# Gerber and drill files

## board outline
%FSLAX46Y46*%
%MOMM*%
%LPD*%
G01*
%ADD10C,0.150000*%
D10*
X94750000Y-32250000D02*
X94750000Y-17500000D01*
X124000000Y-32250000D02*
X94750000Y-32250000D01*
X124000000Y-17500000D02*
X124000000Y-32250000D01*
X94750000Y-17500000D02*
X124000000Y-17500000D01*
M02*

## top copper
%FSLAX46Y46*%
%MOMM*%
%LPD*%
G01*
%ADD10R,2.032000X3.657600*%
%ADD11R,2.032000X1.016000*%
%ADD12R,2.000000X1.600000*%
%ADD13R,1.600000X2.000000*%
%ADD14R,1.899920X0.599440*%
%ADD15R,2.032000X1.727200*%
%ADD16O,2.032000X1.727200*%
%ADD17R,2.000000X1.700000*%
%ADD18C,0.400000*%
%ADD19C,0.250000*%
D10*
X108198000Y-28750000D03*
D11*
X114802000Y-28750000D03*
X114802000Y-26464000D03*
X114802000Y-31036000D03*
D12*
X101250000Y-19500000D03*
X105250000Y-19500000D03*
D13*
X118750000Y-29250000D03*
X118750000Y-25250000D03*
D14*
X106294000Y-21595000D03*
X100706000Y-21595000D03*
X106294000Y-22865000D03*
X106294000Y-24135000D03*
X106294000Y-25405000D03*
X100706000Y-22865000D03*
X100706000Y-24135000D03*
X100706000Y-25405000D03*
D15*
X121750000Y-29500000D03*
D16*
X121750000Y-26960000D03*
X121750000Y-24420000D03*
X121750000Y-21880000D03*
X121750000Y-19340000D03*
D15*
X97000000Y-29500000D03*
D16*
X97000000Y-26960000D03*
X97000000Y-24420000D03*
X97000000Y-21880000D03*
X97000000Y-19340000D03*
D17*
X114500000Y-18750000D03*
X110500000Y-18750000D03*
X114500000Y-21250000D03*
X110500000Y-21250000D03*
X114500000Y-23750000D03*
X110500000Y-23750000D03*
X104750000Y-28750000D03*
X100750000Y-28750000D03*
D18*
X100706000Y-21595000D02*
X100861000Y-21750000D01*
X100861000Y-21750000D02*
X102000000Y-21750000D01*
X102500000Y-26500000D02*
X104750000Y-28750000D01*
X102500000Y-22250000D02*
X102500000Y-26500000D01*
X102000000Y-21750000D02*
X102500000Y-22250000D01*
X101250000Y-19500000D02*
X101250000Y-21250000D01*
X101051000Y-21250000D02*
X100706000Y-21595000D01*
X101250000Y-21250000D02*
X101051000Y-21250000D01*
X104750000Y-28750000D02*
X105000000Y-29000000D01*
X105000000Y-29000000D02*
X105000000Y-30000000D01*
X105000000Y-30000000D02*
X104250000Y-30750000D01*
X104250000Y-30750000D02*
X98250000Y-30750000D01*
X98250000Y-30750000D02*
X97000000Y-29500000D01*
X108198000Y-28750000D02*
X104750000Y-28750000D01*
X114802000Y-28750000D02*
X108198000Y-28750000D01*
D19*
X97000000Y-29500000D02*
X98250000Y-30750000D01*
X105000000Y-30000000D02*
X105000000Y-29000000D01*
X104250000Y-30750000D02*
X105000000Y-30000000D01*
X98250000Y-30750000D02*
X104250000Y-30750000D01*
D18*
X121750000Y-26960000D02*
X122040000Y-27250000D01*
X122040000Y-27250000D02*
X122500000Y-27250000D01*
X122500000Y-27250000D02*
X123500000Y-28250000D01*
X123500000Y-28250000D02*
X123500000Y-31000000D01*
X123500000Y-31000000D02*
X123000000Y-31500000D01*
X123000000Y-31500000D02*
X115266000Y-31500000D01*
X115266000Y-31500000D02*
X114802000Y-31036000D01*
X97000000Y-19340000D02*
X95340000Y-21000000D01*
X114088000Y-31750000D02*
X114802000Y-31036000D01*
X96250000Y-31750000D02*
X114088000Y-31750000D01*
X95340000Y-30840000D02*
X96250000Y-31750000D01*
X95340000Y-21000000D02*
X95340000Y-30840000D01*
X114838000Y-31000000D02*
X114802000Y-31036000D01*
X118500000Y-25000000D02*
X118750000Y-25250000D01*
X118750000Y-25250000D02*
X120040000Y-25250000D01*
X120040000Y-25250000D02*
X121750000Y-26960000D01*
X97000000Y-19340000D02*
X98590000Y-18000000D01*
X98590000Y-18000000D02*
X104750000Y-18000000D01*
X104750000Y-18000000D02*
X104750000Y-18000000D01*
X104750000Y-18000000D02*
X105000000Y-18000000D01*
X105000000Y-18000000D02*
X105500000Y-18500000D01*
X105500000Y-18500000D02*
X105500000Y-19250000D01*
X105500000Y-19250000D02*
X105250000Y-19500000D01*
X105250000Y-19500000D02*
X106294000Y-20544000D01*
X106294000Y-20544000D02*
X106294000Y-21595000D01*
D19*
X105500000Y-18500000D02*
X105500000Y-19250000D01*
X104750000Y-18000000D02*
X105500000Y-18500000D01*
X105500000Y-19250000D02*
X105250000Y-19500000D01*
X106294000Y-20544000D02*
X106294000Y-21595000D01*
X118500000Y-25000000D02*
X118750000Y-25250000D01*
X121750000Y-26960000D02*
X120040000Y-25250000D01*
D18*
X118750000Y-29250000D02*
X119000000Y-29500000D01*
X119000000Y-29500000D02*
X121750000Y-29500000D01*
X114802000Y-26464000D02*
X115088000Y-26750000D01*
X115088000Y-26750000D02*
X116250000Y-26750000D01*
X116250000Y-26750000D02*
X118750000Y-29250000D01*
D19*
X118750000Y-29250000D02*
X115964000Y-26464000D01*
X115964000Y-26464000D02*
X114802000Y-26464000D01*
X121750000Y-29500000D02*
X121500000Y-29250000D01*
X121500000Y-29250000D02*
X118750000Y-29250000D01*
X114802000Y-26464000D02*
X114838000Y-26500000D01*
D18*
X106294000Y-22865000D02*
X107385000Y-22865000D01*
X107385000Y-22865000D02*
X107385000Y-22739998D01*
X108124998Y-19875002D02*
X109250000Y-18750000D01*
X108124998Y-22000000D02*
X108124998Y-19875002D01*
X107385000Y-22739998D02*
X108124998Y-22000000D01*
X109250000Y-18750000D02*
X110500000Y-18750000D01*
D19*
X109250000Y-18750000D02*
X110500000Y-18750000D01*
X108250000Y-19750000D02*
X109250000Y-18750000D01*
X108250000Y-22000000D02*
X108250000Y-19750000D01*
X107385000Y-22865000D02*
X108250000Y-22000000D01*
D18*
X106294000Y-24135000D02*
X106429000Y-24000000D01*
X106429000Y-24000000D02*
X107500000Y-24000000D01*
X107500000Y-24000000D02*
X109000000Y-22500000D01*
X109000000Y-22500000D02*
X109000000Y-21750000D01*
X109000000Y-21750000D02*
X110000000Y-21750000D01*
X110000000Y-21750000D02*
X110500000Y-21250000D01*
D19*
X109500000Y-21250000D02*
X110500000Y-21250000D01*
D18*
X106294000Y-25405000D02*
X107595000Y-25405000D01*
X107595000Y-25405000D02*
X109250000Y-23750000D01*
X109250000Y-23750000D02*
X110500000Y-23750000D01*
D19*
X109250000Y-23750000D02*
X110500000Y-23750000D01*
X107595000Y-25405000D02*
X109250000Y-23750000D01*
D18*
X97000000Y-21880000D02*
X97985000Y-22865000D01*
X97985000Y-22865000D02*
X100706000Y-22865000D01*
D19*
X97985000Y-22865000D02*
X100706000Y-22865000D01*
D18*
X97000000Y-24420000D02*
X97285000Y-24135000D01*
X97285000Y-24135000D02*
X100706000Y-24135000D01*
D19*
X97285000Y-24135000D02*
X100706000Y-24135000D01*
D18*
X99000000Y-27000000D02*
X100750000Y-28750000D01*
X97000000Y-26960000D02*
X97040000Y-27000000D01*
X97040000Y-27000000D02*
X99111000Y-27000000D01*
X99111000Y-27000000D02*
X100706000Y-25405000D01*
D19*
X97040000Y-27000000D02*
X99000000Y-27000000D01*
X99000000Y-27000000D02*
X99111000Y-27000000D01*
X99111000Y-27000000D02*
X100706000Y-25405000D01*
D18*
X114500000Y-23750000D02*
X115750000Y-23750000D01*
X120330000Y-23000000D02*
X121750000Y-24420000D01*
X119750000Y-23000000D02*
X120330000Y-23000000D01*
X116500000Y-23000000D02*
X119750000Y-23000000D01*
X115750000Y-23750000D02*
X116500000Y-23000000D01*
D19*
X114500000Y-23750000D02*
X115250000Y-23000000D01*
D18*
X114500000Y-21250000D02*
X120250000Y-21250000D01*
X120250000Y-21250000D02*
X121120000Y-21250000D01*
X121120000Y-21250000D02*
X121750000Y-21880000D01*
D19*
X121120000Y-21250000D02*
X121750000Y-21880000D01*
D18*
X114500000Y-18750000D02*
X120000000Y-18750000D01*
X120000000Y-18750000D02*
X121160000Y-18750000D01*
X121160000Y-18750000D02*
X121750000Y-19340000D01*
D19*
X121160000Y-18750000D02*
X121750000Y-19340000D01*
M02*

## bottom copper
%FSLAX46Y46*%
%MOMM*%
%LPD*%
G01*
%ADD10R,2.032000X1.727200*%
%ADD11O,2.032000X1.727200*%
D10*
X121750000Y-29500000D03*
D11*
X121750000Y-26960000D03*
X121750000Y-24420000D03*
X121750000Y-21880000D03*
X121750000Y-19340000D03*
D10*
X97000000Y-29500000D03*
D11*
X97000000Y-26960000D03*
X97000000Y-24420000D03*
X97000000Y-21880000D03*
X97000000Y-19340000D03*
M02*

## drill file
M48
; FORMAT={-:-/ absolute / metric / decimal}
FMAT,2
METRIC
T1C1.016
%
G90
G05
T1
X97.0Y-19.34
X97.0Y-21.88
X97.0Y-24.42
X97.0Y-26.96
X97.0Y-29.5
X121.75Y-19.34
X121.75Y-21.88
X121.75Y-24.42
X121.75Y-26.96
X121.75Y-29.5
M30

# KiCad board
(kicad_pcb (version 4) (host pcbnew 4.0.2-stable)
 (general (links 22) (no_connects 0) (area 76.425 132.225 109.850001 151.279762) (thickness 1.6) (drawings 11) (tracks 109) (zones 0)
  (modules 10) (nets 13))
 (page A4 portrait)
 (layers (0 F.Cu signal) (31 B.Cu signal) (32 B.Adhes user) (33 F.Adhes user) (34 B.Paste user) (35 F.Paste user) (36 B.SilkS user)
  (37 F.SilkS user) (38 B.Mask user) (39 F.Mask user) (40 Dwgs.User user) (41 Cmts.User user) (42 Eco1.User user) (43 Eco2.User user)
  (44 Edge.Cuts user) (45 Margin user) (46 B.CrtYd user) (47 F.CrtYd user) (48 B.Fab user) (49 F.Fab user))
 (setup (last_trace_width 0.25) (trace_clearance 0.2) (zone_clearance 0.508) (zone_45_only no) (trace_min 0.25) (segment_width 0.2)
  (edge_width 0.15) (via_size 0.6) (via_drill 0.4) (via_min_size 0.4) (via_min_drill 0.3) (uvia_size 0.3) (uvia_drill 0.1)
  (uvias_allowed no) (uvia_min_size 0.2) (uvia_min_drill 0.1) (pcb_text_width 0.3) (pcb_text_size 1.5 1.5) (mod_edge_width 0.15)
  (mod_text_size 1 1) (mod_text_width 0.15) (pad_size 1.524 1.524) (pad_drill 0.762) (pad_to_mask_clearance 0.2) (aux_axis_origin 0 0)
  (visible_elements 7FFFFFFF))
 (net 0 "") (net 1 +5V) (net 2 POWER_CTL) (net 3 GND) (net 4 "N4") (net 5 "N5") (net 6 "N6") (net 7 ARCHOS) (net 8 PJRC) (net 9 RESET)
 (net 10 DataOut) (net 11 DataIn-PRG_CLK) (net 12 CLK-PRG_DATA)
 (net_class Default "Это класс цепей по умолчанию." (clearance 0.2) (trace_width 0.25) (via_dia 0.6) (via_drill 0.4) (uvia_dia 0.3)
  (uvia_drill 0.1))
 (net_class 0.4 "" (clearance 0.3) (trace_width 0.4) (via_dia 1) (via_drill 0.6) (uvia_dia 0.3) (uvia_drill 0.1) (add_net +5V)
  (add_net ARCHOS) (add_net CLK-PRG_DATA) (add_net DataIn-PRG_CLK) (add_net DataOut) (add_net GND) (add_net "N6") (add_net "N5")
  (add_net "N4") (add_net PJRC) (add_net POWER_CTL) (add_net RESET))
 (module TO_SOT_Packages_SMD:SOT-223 (layer F.Cu) (at 111.5 28.75 90)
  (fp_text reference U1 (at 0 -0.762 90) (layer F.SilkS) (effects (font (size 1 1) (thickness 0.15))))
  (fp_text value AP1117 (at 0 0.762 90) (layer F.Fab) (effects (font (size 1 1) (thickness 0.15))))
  (pad 2 smd rect (at 0 -3.302 90) (size 3.6576 2.032) (layers F.Cu F.Paste F.Mask) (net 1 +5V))
  (pad 2 smd rect (at 0 3.302 90) (size 1.016 2.032) (layers F.Cu F.Paste F.Mask) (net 1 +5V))
  (pad 3 smd rect (at 2.286 3.302 90) (size 1.016 2.032) (layers F.Cu F.Paste F.Mask) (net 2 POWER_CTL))
  (pad 1 smd rect (at -2.286 3.302 90) (size 1.016 2.032) (layers F.Cu F.Paste F.Mask) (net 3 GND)))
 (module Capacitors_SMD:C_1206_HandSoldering (layer F.Cu) (at 103.25 19.5)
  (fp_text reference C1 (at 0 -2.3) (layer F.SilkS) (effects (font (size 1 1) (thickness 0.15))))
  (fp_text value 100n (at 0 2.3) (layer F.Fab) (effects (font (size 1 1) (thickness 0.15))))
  (pad 1 smd rect (at -2 0) (size 2 1.6) (layers F.Cu F.Paste F.Mask) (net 1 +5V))
  (pad 2 smd rect (at 2 0) (size 2 1.6) (layers F.Cu F.Paste F.Mask) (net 3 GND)))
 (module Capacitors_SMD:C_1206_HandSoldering (layer F.Cu) (at 118.75 27.25 90)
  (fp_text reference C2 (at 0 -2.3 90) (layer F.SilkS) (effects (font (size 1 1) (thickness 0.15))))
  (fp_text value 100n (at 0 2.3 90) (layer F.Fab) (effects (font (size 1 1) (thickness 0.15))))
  (pad 1 smd rect (at -2 0 90) (size 2 1.6) (layers F.Cu F.Paste F.Mask) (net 2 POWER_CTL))
  (pad 2 smd rect (at 2 0 90) (size 2 1.6) (layers F.Cu F.Paste F.Mask) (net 3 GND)))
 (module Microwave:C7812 (layer F.Cu) (at 103.5 23.5 270)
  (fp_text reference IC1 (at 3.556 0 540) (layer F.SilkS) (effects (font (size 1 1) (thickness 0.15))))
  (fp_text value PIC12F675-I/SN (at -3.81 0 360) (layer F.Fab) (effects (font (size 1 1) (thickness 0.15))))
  (pad 8 smd rect (at -1.905 -2.794 270) (size 0.59944 1.89992) (layers F.Cu F.Paste F.Mask) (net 3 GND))
  (pad 1 smd rect (at -1.905 2.794 270) (size 0.59944 1.89992) (layers F.Cu F.Paste F.Mask) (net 1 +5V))
  (pad 7 smd rect (at -0.635 -2.794 270) (size 0.59944 1.89992) (layers F.Cu F.Paste F.Mask) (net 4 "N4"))
  (pad 6 smd rect (at 0.635 -2.794 270) (size 0.59944 1.89992) (layers F.Cu F.Paste F.Mask) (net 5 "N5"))
  (pad 5 smd rect (at 1.905 -2.794 270) (size 0.59944 1.89992) (layers F.Cu F.Paste F.Mask) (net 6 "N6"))
  (pad 2 smd rect (at -0.635 2.794 270) (size 0.59944 1.89992) (layers F.Cu F.Paste F.Mask) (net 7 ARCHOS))
  (pad 3 smd rect (at 0.635 2.794 270) (size 0.59944 1.89992) (layers F.Cu F.Paste F.Mask) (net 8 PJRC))
  (pad 4 smd rect (at 1.905 2.794 270) (size 0.59944 1.89992) (layers F.Cu F.Paste F.Mask) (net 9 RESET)))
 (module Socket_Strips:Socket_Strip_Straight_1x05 (layer F.Cu) (at 121.75 29.5 90)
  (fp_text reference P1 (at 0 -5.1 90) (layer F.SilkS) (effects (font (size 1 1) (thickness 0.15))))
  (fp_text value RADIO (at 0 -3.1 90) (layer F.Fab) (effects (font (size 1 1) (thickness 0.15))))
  (pad 1 thru_hole rect (at 0 0 90) (size 1.7272 2.032) (drill 1.016) (layers *.Cu *.Mask F.SilkS) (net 2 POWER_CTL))
  (pad 2 thru_hole oval (at 2.54 0 90) (size 1.7272 2.032) (drill 1.016) (layers *.Cu *.Mask F.SilkS) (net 3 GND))
  (pad 3 thru_hole oval (at 5.08 0 90) (size 1.7272 2.032) (drill 1.016) (layers *.Cu *.Mask F.SilkS) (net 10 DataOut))
  (pad 4 thru_hole oval (at 7.62 0 90) (size 1.7272 2.032) (drill 1.016) (layers *.Cu *.Mask F.SilkS) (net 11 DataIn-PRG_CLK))
  (pad 5 thru_hole oval (at 10.16 0 90) (size 1.7272 2.032) (drill 1.016) (layers *.Cu *.Mask F.SilkS) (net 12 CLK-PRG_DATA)))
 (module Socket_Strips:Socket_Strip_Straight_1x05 (layer F.Cu) (at 97 29.5 90)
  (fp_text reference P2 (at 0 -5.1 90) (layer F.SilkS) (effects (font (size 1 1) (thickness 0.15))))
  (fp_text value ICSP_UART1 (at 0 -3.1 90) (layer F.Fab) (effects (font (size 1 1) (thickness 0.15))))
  (pad 1 thru_hole rect (at 0 0 90) (size 1.7272 2.032) (drill 1.016) (layers *.Cu *.Mask F.SilkS) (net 1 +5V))
  (pad 2 thru_hole oval (at 2.54 0 90) (size 1.7272 2.032) (drill 1.016) (layers *.Cu *.Mask F.SilkS) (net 9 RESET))
  (pad 3 thru_hole oval (at 5.08 0 90) (size 1.7272 2.032) (drill 1.016) (layers *.Cu *.Mask F.SilkS) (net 8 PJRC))
  (pad 4 thru_hole oval (at 7.62 0 90) (size 1.7272 2.032) (drill 1.016) (layers *.Cu *.Mask F.SilkS) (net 7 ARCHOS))
  (pad 5 thru_hole oval (at 10.16 0 90) (size 1.7272 2.032) (drill 1.016) (layers *.Cu *.Mask F.SilkS) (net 3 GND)))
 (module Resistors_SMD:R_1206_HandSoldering (layer F.Cu) (at 112.5 18.75 180)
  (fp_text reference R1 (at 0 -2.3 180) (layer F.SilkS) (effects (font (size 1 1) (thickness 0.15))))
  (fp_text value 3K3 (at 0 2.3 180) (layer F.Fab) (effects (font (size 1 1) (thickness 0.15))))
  (pad 1 smd rect (at -2 0 180) (size 2 1.7) (layers F.Cu F.Paste F.Mask) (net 12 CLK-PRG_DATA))
  (pad 2 smd rect (at 2 0 180) (size 2 1.7) (layers F.Cu F.Paste F.Mask) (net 4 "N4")))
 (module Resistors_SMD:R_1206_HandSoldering (layer F.Cu) (at 112.5 21.25 180)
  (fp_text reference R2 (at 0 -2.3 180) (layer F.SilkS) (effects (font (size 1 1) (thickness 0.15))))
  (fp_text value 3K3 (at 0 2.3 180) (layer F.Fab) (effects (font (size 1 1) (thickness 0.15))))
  (pad 1 smd rect (at -2 0 180) (size 2 1.7) (layers F.Cu F.Paste F.Mask) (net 11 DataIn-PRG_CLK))
  (pad 2 smd rect (at 2 0 180) (size 2 1.7) (layers F.Cu F.Paste F.Mask) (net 5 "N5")))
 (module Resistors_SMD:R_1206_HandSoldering (layer F.Cu) (at 112.5 23.75 180)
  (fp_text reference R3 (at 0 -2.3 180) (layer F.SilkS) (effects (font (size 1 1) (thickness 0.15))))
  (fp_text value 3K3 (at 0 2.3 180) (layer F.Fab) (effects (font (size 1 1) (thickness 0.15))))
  (pad 1 smd rect (at -2 0 180) (size 2 1.7) (layers F.Cu F.Paste F.Mask) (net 10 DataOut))
  (pad 2 smd rect (at 2 0 180) (size 2 1.7) (layers F.Cu F.Paste F.Mask) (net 6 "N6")))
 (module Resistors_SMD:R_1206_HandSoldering (layer F.Cu) (at 102.75 28.75 180)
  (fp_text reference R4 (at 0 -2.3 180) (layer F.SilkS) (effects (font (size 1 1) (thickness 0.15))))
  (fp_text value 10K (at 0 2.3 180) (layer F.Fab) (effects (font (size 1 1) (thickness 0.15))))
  (pad 1 smd rect (at -2 0 180) (size 2 1.7) (layers F.Cu F.Paste F.Mask) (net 1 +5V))
  (pad 2 smd rect (at 2 0 180) (size 2 1.7) (layers F.Cu F.Paste F.Mask) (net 9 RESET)))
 (gr_line (start 94.75 32.25) (end 94.75 17.5) (angle 90) (layer Edge.Cuts) (width 0.15))
 (gr_line (start 124 32.25) (end 94.75 32.25) (angle 90) (layer Edge.Cuts) (width 0.15))
 (gr_line (start 124 17.5) (end 124 32.25) (angle 90) (layer Edge.Cuts) (width 0.15))
 (gr_line (start 94.75 17.5) (end 124 17.5) (angle 90) (layer Edge.Cuts) (width 0.15))
 (segment (start 100.706 21.595) (end 100.861 21.75) (width 0.4) (layer F.Cu) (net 1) (status 30))
 (segment (start 100.861 21.75) (end 102 21.75) (width 0.4) (layer F.Cu) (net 1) (status 10))
 (segment (start 102.5 26.5) (end 104.75 28.75) (width 0.4) (layer F.Cu) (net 1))
 (segment (start 102.5 22.25) (end 102.5 26.5) (width 0.4) (layer F.Cu) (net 1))
 (segment (start 102 21.75) (end 102.5 22.25) (width 0.4) (layer F.Cu) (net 1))
 (segment (start 101.25 19.5) (end 101.25 21.25) (width 0.4) (layer F.Cu) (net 1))
 (segment (start 101.051 21.25) (end 100.706 21.595) (width 0.4) (layer F.Cu) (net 1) (status 20))
 (segment (start 101.25 21.25) (end 101.051 21.25) (width 0.4) (layer F.Cu) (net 1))
 (segment (start 104.75 28.75) (end 105 29) (width 0.4) (layer F.Cu) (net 1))
 (segment (start 105 29) (end 105 30) (width 0.4) (layer F.Cu) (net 1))
 (segment (start 105 30) (end 104.25 30.75) (width 0.4) (layer F.Cu) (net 1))
 (segment (start 104.25 30.75) (end 98.25 30.75) (width 0.4) (layer F.Cu) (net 1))
 (segment (start 98.25 30.75) (end 97 29.5) (width 0.4) (layer F.Cu) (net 1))
 (segment (start 108.198 28.75) (end 104.75 28.75) (width 0.4) (layer F.Cu) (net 1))
 (segment (start 114.802 28.75) (end 108.198 28.75) (width 0.4) (layer F.Cu) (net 1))
 (segment (start 97 29.5) (end 98.25 30.75) (width 0.25) (layer F.Cu) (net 1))
 (segment (start 105 30) (end 105 29) (width 0.25) (layer F.Cu) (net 1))
 (segment (start 104.25 30.75) (end 105 30) (width 0.25) (layer F.Cu) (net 1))
 (segment (start 98.25 30.75) (end 104.25 30.75) (width 0.25) (layer F.Cu) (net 1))
 (segment (start 121.75 26.96) (end 122.04 27.25) (width 0.4) (layer F.Cu) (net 3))
 (segment (start 122.04 27.25) (end 122.5 27.25) (width 0.4) (layer F.Cu) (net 3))
 (segment (start 122.5 27.25) (end 123.5 28.25) (width 0.4) (layer F.Cu) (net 3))
 (segment (start 123.5 28.25) (end 123.5 31) (width 0.4) (layer F.Cu) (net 3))
 (segment (start 123.5 31) (end 123 31.5) (width 0.4) (layer F.Cu) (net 3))
 (segment (start 123 31.5) (end 115.266 31.5) (width 0.4) (layer F.Cu) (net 3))
 (segment (start 115.266 31.5) (end 114.802 31.036) (width 0.4) (layer F.Cu) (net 3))
 (segment (start 97 19.34) (end 95.34 21) (width 0.4) (layer F.Cu) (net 3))
 (segment (start 114.088 31.75) (end 114.802 31.036) (width 0.4) (layer F.Cu) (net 3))
 (segment (start 96.25 31.75) (end 114.088 31.75) (width 0.4) (layer F.Cu) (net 3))
 (segment (start 95.34 30.84) (end 96.25 31.75) (width 0.4) (layer F.Cu) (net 3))
 (segment (start 95.34 21) (end 95.34 30.84) (width 0.4) (layer F.Cu) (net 3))
 (segment (start 114.838 31) (end 114.802 31.036) (width 0.4) (layer F.Cu) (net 3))
 (segment (start 118.5 25) (end 118.75 25.25) (width 0.4) (layer F.Cu) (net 3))
 (segment (start 118.75 25.25) (end 120.04 25.25) (width 0.4) (layer F.Cu) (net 3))
 (segment (start 120.04 25.25) (end 121.75 26.96) (width 0.4) (layer F.Cu) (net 3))
 (segment (start 97 19.34) (end 98.59 18) (width 0.4) (layer F.Cu) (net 3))
 (segment (start 98.59 18) (end 104.75 18) (width 0.4) (layer F.Cu) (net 3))
 (segment (start 104.75 18) (end 104.75 18) (width 0.4) (layer F.Cu) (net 3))
 (segment (start 104.75 18) (end 105 18) (width 0.4) (layer F.Cu) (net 3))
 (segment (start 105 18) (end 105.5 18.5) (width 0.4) (layer F.Cu) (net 3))
 (segment (start 105.5 18.5) (end 105.5 19.25) (width 0.4) (layer F.Cu) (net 3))
 (segment (start 105.5 19.25) (end 105.25 19.5) (width 0.4) (layer F.Cu) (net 3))
 (segment (start 105.25 19.5) (end 106.294 20.544) (width 0.4) (layer F.Cu) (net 3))
 (segment (start 106.294 20.544) (end 106.294 21.595) (width 0.4) (layer F.Cu) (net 3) (status 20))
 (segment (start 105.5 18.5) (end 105.5 19.25) (width 0.25) (layer F.Cu) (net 3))
 (segment (start 104.75 18) (end 105.5 18.5) (width 0.25) (layer F.Cu) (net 3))
 (segment (start 105.5 19.25) (end 105.25 19.5) (width 0.25) (layer F.Cu) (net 3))
 (segment (start 106.294 20.544) (end 106.294 21.595) (width 0.25) (layer F.Cu) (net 3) (status 20))
 (segment (start 118.5 25) (end 118.75 25.25) (width 0.25) (layer F.Cu) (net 3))
 (segment (start 121.75 26.96) (end 120.04 25.25) (width 0.25) (layer F.Cu) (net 3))
 (segment (start 118.75 29.25) (end 119 29.5) (width 0.4) (layer F.Cu) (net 2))
 (segment (start 119 29.5) (end 121.75 29.5) (width 0.4) (layer F.Cu) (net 2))
 (segment (start 114.802 26.464) (end 115.088 26.75) (width 0.4) (layer F.Cu) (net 2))
 (segment (start 115.088 26.75) (end 116.25 26.75) (width 0.4) (layer F.Cu) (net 2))
 (segment (start 116.25 26.75) (end 118.75 29.25) (width 0.4) (layer F.Cu) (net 2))
 (segment (start 118.75 29.25) (end 115.964 26.464) (width 0.25) (layer F.Cu) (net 2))
 (segment (start 115.964 26.464) (end 114.802 26.464) (width 0.25) (layer F.Cu) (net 2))
 (segment (start 121.75 29.5) (end 121.5 29.25) (width 0.25) (layer F.Cu) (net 2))
 (segment (start 121.5 29.25) (end 118.75 29.25) (width 0.25) (layer F.Cu) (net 2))
 (segment (start 114.802 26.464) (end 114.838 26.5) (width 0.25) (layer F.Cu) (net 2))
 (segment (start 106.294 22.865) (end 107.385 22.865) (width 0.4) (layer F.Cu) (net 4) (status 10))
 (segment (start 107.385 22.865) (end 107.385 22.739998) (width 0.4) (layer F.Cu) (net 4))
 (segment (start 108.124998 19.875002) (end 109.25 18.75) (width 0.4) (layer F.Cu) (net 4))
 (segment (start 108.124998 22) (end 108.124998 19.875002) (width 0.4) (layer F.Cu) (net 4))
 (segment (start 107.385 22.739998) (end 108.124998 22) (width 0.4) (layer F.Cu) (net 4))
 (segment (start 109.25 18.75) (end 110.5 18.75) (width 0.4) (layer F.Cu) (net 4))
 (segment (start 109.25 18.75) (end 110.5 18.75) (width 0.25) (layer F.Cu) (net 4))
 (segment (start 108.25 19.75) (end 109.25 18.75) (width 0.25) (layer F.Cu) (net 4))
 (segment (start 108.25 22) (end 108.25 19.75) (width 0.25) (layer F.Cu) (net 4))
 (segment (start 107.385 22.865) (end 108.25 22) (width 0.25) (layer F.Cu) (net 4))
 (segment (start 106.294 24.135) (end 106.429 24) (width 0.4) (layer F.Cu) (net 5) (status 30))
 (segment (start 106.429 24) (end 107.5 24) (width 0.4) (layer F.Cu) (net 5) (status 10))
 (segment (start 107.5 24) (end 109 22.5) (width 0.4) (layer F.Cu) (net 5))
 (segment (start 109 22.5) (end 109 21.75) (width 0.4) (layer F.Cu) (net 5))
 (segment (start 109 21.75) (end 110 21.75) (width 0.4) (layer F.Cu) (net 5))
 (segment (start 110 21.75) (end 110.5 21.25) (width 0.4) (layer F.Cu) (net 5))
 (segment (start 109.5 21.25) (end 110.5 21.25) (width 0.25) (layer F.Cu) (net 5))
 (segment (start 106.294 25.405) (end 107.595 25.405) (width 0.4) (layer F.Cu) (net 6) (status 10))
 (segment (start 107.595 25.405) (end 109.25 23.75) (width 0.4) (layer F.Cu) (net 6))
 (segment (start 109.25 23.75) (end 110.5 23.75) (width 0.4) (layer F.Cu) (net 6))
 (segment (start 109.25 23.75) (end 110.5 23.75) (width 0.25) (layer F.Cu) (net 6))
 (segment (start 107.595 25.405) (end 109.25 23.75) (width 0.25) (layer F.Cu) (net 6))
 (segment (start 97 21.88) (end 97.985 22.865) (width 0.4) (layer F.Cu) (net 7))
 (segment (start 97.985 22.865) (end 100.706 22.865) (width 0.4) (layer F.Cu) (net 7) (status 20))
 (segment (start 97.985 22.865) (end 100.706 22.865) (width 0.25) (layer F.Cu) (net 7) (status 20))
 (segment (start 97 24.42) (end 97.285 24.135) (width 0.4) (layer F.Cu) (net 8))
 (segment (start 97.285 24.135) (end 100.706 24.135) (width 0.4) (layer F.Cu) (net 8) (status 20))
 (segment (start 97.285 24.135) (end 100.706 24.135) (width 0.25) (layer F.Cu) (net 8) (status 20))
 (segment (start 99 27) (end 100.75 28.75) (width 0.4) (layer F.Cu) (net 9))
 (segment (start 97 26.96) (end 97.04 27) (width 0.4) (layer F.Cu) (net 9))
 (segment (start 97.04 27) (end 99.111 27) (width 0.4) (layer F.Cu) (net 9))
 (segment (start 99.111 27) (end 100.706 25.405) (width 0.4) (layer F.Cu) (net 9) (status 20))
 (segment (start 97.04 27) (end 99 27) (width 0.25) (layer F.Cu) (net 9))
 (segment (start 99 27) (end 99.111 27) (width 0.25) (layer F.Cu) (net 9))
 (segment (start 99.111 27) (end 100.706 25.405) (width 0.25) (layer F.Cu) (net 9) (status 20))
 (segment (start 114.5 23.75) (end 115.75 23.75) (width 0.4) (layer F.Cu) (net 10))
 (segment (start 120.33 23) (end 121.75 24.42) (width 0.4) (layer F.Cu) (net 10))
 (segment (start 119.75 23) (end 120.33 23) (width 0.4) (layer F.Cu) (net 10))
 (segment (start 116.5 23) (end 119.75 23) (width 0.4) (layer F.Cu) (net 10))
 (segment (start 115.75 23.75) (end 116.5 23) (width 0.4) (layer F.Cu) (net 10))
 (segment (start 114.5 23.75) (end 115.25 23) (width 0.25) (layer F.Cu) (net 10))
 (segment (start 114.5 21.25) (end 120.25 21.25) (width 0.4) (layer F.Cu) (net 11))
 (segment (start 120.25 21.25) (end 121.12 21.25) (width 0.4) (layer F.Cu) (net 11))
 (segment (start 121.12 21.25) (end 121.75 21.88) (width 0.4) (layer F.Cu) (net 11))
 (segment (start 121.12 21.25) (end 121.75 21.88) (width 0.25) (layer F.Cu) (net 11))
 (segment (start 114.5 18.75) (end 120 18.75) (width 0.4) (layer F.Cu) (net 12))
 (segment (start 120 18.75) (end 121.16 18.75) (width 0.4) (layer F.Cu) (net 12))
 (segment (start 121.16 18.75) (end 121.75 19.34) (width 0.4) (layer F.Cu) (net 12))
 (segment (start 121.16 18.75) (end 121.75 19.34) (width 0.25) (layer F.Cu) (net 12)))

